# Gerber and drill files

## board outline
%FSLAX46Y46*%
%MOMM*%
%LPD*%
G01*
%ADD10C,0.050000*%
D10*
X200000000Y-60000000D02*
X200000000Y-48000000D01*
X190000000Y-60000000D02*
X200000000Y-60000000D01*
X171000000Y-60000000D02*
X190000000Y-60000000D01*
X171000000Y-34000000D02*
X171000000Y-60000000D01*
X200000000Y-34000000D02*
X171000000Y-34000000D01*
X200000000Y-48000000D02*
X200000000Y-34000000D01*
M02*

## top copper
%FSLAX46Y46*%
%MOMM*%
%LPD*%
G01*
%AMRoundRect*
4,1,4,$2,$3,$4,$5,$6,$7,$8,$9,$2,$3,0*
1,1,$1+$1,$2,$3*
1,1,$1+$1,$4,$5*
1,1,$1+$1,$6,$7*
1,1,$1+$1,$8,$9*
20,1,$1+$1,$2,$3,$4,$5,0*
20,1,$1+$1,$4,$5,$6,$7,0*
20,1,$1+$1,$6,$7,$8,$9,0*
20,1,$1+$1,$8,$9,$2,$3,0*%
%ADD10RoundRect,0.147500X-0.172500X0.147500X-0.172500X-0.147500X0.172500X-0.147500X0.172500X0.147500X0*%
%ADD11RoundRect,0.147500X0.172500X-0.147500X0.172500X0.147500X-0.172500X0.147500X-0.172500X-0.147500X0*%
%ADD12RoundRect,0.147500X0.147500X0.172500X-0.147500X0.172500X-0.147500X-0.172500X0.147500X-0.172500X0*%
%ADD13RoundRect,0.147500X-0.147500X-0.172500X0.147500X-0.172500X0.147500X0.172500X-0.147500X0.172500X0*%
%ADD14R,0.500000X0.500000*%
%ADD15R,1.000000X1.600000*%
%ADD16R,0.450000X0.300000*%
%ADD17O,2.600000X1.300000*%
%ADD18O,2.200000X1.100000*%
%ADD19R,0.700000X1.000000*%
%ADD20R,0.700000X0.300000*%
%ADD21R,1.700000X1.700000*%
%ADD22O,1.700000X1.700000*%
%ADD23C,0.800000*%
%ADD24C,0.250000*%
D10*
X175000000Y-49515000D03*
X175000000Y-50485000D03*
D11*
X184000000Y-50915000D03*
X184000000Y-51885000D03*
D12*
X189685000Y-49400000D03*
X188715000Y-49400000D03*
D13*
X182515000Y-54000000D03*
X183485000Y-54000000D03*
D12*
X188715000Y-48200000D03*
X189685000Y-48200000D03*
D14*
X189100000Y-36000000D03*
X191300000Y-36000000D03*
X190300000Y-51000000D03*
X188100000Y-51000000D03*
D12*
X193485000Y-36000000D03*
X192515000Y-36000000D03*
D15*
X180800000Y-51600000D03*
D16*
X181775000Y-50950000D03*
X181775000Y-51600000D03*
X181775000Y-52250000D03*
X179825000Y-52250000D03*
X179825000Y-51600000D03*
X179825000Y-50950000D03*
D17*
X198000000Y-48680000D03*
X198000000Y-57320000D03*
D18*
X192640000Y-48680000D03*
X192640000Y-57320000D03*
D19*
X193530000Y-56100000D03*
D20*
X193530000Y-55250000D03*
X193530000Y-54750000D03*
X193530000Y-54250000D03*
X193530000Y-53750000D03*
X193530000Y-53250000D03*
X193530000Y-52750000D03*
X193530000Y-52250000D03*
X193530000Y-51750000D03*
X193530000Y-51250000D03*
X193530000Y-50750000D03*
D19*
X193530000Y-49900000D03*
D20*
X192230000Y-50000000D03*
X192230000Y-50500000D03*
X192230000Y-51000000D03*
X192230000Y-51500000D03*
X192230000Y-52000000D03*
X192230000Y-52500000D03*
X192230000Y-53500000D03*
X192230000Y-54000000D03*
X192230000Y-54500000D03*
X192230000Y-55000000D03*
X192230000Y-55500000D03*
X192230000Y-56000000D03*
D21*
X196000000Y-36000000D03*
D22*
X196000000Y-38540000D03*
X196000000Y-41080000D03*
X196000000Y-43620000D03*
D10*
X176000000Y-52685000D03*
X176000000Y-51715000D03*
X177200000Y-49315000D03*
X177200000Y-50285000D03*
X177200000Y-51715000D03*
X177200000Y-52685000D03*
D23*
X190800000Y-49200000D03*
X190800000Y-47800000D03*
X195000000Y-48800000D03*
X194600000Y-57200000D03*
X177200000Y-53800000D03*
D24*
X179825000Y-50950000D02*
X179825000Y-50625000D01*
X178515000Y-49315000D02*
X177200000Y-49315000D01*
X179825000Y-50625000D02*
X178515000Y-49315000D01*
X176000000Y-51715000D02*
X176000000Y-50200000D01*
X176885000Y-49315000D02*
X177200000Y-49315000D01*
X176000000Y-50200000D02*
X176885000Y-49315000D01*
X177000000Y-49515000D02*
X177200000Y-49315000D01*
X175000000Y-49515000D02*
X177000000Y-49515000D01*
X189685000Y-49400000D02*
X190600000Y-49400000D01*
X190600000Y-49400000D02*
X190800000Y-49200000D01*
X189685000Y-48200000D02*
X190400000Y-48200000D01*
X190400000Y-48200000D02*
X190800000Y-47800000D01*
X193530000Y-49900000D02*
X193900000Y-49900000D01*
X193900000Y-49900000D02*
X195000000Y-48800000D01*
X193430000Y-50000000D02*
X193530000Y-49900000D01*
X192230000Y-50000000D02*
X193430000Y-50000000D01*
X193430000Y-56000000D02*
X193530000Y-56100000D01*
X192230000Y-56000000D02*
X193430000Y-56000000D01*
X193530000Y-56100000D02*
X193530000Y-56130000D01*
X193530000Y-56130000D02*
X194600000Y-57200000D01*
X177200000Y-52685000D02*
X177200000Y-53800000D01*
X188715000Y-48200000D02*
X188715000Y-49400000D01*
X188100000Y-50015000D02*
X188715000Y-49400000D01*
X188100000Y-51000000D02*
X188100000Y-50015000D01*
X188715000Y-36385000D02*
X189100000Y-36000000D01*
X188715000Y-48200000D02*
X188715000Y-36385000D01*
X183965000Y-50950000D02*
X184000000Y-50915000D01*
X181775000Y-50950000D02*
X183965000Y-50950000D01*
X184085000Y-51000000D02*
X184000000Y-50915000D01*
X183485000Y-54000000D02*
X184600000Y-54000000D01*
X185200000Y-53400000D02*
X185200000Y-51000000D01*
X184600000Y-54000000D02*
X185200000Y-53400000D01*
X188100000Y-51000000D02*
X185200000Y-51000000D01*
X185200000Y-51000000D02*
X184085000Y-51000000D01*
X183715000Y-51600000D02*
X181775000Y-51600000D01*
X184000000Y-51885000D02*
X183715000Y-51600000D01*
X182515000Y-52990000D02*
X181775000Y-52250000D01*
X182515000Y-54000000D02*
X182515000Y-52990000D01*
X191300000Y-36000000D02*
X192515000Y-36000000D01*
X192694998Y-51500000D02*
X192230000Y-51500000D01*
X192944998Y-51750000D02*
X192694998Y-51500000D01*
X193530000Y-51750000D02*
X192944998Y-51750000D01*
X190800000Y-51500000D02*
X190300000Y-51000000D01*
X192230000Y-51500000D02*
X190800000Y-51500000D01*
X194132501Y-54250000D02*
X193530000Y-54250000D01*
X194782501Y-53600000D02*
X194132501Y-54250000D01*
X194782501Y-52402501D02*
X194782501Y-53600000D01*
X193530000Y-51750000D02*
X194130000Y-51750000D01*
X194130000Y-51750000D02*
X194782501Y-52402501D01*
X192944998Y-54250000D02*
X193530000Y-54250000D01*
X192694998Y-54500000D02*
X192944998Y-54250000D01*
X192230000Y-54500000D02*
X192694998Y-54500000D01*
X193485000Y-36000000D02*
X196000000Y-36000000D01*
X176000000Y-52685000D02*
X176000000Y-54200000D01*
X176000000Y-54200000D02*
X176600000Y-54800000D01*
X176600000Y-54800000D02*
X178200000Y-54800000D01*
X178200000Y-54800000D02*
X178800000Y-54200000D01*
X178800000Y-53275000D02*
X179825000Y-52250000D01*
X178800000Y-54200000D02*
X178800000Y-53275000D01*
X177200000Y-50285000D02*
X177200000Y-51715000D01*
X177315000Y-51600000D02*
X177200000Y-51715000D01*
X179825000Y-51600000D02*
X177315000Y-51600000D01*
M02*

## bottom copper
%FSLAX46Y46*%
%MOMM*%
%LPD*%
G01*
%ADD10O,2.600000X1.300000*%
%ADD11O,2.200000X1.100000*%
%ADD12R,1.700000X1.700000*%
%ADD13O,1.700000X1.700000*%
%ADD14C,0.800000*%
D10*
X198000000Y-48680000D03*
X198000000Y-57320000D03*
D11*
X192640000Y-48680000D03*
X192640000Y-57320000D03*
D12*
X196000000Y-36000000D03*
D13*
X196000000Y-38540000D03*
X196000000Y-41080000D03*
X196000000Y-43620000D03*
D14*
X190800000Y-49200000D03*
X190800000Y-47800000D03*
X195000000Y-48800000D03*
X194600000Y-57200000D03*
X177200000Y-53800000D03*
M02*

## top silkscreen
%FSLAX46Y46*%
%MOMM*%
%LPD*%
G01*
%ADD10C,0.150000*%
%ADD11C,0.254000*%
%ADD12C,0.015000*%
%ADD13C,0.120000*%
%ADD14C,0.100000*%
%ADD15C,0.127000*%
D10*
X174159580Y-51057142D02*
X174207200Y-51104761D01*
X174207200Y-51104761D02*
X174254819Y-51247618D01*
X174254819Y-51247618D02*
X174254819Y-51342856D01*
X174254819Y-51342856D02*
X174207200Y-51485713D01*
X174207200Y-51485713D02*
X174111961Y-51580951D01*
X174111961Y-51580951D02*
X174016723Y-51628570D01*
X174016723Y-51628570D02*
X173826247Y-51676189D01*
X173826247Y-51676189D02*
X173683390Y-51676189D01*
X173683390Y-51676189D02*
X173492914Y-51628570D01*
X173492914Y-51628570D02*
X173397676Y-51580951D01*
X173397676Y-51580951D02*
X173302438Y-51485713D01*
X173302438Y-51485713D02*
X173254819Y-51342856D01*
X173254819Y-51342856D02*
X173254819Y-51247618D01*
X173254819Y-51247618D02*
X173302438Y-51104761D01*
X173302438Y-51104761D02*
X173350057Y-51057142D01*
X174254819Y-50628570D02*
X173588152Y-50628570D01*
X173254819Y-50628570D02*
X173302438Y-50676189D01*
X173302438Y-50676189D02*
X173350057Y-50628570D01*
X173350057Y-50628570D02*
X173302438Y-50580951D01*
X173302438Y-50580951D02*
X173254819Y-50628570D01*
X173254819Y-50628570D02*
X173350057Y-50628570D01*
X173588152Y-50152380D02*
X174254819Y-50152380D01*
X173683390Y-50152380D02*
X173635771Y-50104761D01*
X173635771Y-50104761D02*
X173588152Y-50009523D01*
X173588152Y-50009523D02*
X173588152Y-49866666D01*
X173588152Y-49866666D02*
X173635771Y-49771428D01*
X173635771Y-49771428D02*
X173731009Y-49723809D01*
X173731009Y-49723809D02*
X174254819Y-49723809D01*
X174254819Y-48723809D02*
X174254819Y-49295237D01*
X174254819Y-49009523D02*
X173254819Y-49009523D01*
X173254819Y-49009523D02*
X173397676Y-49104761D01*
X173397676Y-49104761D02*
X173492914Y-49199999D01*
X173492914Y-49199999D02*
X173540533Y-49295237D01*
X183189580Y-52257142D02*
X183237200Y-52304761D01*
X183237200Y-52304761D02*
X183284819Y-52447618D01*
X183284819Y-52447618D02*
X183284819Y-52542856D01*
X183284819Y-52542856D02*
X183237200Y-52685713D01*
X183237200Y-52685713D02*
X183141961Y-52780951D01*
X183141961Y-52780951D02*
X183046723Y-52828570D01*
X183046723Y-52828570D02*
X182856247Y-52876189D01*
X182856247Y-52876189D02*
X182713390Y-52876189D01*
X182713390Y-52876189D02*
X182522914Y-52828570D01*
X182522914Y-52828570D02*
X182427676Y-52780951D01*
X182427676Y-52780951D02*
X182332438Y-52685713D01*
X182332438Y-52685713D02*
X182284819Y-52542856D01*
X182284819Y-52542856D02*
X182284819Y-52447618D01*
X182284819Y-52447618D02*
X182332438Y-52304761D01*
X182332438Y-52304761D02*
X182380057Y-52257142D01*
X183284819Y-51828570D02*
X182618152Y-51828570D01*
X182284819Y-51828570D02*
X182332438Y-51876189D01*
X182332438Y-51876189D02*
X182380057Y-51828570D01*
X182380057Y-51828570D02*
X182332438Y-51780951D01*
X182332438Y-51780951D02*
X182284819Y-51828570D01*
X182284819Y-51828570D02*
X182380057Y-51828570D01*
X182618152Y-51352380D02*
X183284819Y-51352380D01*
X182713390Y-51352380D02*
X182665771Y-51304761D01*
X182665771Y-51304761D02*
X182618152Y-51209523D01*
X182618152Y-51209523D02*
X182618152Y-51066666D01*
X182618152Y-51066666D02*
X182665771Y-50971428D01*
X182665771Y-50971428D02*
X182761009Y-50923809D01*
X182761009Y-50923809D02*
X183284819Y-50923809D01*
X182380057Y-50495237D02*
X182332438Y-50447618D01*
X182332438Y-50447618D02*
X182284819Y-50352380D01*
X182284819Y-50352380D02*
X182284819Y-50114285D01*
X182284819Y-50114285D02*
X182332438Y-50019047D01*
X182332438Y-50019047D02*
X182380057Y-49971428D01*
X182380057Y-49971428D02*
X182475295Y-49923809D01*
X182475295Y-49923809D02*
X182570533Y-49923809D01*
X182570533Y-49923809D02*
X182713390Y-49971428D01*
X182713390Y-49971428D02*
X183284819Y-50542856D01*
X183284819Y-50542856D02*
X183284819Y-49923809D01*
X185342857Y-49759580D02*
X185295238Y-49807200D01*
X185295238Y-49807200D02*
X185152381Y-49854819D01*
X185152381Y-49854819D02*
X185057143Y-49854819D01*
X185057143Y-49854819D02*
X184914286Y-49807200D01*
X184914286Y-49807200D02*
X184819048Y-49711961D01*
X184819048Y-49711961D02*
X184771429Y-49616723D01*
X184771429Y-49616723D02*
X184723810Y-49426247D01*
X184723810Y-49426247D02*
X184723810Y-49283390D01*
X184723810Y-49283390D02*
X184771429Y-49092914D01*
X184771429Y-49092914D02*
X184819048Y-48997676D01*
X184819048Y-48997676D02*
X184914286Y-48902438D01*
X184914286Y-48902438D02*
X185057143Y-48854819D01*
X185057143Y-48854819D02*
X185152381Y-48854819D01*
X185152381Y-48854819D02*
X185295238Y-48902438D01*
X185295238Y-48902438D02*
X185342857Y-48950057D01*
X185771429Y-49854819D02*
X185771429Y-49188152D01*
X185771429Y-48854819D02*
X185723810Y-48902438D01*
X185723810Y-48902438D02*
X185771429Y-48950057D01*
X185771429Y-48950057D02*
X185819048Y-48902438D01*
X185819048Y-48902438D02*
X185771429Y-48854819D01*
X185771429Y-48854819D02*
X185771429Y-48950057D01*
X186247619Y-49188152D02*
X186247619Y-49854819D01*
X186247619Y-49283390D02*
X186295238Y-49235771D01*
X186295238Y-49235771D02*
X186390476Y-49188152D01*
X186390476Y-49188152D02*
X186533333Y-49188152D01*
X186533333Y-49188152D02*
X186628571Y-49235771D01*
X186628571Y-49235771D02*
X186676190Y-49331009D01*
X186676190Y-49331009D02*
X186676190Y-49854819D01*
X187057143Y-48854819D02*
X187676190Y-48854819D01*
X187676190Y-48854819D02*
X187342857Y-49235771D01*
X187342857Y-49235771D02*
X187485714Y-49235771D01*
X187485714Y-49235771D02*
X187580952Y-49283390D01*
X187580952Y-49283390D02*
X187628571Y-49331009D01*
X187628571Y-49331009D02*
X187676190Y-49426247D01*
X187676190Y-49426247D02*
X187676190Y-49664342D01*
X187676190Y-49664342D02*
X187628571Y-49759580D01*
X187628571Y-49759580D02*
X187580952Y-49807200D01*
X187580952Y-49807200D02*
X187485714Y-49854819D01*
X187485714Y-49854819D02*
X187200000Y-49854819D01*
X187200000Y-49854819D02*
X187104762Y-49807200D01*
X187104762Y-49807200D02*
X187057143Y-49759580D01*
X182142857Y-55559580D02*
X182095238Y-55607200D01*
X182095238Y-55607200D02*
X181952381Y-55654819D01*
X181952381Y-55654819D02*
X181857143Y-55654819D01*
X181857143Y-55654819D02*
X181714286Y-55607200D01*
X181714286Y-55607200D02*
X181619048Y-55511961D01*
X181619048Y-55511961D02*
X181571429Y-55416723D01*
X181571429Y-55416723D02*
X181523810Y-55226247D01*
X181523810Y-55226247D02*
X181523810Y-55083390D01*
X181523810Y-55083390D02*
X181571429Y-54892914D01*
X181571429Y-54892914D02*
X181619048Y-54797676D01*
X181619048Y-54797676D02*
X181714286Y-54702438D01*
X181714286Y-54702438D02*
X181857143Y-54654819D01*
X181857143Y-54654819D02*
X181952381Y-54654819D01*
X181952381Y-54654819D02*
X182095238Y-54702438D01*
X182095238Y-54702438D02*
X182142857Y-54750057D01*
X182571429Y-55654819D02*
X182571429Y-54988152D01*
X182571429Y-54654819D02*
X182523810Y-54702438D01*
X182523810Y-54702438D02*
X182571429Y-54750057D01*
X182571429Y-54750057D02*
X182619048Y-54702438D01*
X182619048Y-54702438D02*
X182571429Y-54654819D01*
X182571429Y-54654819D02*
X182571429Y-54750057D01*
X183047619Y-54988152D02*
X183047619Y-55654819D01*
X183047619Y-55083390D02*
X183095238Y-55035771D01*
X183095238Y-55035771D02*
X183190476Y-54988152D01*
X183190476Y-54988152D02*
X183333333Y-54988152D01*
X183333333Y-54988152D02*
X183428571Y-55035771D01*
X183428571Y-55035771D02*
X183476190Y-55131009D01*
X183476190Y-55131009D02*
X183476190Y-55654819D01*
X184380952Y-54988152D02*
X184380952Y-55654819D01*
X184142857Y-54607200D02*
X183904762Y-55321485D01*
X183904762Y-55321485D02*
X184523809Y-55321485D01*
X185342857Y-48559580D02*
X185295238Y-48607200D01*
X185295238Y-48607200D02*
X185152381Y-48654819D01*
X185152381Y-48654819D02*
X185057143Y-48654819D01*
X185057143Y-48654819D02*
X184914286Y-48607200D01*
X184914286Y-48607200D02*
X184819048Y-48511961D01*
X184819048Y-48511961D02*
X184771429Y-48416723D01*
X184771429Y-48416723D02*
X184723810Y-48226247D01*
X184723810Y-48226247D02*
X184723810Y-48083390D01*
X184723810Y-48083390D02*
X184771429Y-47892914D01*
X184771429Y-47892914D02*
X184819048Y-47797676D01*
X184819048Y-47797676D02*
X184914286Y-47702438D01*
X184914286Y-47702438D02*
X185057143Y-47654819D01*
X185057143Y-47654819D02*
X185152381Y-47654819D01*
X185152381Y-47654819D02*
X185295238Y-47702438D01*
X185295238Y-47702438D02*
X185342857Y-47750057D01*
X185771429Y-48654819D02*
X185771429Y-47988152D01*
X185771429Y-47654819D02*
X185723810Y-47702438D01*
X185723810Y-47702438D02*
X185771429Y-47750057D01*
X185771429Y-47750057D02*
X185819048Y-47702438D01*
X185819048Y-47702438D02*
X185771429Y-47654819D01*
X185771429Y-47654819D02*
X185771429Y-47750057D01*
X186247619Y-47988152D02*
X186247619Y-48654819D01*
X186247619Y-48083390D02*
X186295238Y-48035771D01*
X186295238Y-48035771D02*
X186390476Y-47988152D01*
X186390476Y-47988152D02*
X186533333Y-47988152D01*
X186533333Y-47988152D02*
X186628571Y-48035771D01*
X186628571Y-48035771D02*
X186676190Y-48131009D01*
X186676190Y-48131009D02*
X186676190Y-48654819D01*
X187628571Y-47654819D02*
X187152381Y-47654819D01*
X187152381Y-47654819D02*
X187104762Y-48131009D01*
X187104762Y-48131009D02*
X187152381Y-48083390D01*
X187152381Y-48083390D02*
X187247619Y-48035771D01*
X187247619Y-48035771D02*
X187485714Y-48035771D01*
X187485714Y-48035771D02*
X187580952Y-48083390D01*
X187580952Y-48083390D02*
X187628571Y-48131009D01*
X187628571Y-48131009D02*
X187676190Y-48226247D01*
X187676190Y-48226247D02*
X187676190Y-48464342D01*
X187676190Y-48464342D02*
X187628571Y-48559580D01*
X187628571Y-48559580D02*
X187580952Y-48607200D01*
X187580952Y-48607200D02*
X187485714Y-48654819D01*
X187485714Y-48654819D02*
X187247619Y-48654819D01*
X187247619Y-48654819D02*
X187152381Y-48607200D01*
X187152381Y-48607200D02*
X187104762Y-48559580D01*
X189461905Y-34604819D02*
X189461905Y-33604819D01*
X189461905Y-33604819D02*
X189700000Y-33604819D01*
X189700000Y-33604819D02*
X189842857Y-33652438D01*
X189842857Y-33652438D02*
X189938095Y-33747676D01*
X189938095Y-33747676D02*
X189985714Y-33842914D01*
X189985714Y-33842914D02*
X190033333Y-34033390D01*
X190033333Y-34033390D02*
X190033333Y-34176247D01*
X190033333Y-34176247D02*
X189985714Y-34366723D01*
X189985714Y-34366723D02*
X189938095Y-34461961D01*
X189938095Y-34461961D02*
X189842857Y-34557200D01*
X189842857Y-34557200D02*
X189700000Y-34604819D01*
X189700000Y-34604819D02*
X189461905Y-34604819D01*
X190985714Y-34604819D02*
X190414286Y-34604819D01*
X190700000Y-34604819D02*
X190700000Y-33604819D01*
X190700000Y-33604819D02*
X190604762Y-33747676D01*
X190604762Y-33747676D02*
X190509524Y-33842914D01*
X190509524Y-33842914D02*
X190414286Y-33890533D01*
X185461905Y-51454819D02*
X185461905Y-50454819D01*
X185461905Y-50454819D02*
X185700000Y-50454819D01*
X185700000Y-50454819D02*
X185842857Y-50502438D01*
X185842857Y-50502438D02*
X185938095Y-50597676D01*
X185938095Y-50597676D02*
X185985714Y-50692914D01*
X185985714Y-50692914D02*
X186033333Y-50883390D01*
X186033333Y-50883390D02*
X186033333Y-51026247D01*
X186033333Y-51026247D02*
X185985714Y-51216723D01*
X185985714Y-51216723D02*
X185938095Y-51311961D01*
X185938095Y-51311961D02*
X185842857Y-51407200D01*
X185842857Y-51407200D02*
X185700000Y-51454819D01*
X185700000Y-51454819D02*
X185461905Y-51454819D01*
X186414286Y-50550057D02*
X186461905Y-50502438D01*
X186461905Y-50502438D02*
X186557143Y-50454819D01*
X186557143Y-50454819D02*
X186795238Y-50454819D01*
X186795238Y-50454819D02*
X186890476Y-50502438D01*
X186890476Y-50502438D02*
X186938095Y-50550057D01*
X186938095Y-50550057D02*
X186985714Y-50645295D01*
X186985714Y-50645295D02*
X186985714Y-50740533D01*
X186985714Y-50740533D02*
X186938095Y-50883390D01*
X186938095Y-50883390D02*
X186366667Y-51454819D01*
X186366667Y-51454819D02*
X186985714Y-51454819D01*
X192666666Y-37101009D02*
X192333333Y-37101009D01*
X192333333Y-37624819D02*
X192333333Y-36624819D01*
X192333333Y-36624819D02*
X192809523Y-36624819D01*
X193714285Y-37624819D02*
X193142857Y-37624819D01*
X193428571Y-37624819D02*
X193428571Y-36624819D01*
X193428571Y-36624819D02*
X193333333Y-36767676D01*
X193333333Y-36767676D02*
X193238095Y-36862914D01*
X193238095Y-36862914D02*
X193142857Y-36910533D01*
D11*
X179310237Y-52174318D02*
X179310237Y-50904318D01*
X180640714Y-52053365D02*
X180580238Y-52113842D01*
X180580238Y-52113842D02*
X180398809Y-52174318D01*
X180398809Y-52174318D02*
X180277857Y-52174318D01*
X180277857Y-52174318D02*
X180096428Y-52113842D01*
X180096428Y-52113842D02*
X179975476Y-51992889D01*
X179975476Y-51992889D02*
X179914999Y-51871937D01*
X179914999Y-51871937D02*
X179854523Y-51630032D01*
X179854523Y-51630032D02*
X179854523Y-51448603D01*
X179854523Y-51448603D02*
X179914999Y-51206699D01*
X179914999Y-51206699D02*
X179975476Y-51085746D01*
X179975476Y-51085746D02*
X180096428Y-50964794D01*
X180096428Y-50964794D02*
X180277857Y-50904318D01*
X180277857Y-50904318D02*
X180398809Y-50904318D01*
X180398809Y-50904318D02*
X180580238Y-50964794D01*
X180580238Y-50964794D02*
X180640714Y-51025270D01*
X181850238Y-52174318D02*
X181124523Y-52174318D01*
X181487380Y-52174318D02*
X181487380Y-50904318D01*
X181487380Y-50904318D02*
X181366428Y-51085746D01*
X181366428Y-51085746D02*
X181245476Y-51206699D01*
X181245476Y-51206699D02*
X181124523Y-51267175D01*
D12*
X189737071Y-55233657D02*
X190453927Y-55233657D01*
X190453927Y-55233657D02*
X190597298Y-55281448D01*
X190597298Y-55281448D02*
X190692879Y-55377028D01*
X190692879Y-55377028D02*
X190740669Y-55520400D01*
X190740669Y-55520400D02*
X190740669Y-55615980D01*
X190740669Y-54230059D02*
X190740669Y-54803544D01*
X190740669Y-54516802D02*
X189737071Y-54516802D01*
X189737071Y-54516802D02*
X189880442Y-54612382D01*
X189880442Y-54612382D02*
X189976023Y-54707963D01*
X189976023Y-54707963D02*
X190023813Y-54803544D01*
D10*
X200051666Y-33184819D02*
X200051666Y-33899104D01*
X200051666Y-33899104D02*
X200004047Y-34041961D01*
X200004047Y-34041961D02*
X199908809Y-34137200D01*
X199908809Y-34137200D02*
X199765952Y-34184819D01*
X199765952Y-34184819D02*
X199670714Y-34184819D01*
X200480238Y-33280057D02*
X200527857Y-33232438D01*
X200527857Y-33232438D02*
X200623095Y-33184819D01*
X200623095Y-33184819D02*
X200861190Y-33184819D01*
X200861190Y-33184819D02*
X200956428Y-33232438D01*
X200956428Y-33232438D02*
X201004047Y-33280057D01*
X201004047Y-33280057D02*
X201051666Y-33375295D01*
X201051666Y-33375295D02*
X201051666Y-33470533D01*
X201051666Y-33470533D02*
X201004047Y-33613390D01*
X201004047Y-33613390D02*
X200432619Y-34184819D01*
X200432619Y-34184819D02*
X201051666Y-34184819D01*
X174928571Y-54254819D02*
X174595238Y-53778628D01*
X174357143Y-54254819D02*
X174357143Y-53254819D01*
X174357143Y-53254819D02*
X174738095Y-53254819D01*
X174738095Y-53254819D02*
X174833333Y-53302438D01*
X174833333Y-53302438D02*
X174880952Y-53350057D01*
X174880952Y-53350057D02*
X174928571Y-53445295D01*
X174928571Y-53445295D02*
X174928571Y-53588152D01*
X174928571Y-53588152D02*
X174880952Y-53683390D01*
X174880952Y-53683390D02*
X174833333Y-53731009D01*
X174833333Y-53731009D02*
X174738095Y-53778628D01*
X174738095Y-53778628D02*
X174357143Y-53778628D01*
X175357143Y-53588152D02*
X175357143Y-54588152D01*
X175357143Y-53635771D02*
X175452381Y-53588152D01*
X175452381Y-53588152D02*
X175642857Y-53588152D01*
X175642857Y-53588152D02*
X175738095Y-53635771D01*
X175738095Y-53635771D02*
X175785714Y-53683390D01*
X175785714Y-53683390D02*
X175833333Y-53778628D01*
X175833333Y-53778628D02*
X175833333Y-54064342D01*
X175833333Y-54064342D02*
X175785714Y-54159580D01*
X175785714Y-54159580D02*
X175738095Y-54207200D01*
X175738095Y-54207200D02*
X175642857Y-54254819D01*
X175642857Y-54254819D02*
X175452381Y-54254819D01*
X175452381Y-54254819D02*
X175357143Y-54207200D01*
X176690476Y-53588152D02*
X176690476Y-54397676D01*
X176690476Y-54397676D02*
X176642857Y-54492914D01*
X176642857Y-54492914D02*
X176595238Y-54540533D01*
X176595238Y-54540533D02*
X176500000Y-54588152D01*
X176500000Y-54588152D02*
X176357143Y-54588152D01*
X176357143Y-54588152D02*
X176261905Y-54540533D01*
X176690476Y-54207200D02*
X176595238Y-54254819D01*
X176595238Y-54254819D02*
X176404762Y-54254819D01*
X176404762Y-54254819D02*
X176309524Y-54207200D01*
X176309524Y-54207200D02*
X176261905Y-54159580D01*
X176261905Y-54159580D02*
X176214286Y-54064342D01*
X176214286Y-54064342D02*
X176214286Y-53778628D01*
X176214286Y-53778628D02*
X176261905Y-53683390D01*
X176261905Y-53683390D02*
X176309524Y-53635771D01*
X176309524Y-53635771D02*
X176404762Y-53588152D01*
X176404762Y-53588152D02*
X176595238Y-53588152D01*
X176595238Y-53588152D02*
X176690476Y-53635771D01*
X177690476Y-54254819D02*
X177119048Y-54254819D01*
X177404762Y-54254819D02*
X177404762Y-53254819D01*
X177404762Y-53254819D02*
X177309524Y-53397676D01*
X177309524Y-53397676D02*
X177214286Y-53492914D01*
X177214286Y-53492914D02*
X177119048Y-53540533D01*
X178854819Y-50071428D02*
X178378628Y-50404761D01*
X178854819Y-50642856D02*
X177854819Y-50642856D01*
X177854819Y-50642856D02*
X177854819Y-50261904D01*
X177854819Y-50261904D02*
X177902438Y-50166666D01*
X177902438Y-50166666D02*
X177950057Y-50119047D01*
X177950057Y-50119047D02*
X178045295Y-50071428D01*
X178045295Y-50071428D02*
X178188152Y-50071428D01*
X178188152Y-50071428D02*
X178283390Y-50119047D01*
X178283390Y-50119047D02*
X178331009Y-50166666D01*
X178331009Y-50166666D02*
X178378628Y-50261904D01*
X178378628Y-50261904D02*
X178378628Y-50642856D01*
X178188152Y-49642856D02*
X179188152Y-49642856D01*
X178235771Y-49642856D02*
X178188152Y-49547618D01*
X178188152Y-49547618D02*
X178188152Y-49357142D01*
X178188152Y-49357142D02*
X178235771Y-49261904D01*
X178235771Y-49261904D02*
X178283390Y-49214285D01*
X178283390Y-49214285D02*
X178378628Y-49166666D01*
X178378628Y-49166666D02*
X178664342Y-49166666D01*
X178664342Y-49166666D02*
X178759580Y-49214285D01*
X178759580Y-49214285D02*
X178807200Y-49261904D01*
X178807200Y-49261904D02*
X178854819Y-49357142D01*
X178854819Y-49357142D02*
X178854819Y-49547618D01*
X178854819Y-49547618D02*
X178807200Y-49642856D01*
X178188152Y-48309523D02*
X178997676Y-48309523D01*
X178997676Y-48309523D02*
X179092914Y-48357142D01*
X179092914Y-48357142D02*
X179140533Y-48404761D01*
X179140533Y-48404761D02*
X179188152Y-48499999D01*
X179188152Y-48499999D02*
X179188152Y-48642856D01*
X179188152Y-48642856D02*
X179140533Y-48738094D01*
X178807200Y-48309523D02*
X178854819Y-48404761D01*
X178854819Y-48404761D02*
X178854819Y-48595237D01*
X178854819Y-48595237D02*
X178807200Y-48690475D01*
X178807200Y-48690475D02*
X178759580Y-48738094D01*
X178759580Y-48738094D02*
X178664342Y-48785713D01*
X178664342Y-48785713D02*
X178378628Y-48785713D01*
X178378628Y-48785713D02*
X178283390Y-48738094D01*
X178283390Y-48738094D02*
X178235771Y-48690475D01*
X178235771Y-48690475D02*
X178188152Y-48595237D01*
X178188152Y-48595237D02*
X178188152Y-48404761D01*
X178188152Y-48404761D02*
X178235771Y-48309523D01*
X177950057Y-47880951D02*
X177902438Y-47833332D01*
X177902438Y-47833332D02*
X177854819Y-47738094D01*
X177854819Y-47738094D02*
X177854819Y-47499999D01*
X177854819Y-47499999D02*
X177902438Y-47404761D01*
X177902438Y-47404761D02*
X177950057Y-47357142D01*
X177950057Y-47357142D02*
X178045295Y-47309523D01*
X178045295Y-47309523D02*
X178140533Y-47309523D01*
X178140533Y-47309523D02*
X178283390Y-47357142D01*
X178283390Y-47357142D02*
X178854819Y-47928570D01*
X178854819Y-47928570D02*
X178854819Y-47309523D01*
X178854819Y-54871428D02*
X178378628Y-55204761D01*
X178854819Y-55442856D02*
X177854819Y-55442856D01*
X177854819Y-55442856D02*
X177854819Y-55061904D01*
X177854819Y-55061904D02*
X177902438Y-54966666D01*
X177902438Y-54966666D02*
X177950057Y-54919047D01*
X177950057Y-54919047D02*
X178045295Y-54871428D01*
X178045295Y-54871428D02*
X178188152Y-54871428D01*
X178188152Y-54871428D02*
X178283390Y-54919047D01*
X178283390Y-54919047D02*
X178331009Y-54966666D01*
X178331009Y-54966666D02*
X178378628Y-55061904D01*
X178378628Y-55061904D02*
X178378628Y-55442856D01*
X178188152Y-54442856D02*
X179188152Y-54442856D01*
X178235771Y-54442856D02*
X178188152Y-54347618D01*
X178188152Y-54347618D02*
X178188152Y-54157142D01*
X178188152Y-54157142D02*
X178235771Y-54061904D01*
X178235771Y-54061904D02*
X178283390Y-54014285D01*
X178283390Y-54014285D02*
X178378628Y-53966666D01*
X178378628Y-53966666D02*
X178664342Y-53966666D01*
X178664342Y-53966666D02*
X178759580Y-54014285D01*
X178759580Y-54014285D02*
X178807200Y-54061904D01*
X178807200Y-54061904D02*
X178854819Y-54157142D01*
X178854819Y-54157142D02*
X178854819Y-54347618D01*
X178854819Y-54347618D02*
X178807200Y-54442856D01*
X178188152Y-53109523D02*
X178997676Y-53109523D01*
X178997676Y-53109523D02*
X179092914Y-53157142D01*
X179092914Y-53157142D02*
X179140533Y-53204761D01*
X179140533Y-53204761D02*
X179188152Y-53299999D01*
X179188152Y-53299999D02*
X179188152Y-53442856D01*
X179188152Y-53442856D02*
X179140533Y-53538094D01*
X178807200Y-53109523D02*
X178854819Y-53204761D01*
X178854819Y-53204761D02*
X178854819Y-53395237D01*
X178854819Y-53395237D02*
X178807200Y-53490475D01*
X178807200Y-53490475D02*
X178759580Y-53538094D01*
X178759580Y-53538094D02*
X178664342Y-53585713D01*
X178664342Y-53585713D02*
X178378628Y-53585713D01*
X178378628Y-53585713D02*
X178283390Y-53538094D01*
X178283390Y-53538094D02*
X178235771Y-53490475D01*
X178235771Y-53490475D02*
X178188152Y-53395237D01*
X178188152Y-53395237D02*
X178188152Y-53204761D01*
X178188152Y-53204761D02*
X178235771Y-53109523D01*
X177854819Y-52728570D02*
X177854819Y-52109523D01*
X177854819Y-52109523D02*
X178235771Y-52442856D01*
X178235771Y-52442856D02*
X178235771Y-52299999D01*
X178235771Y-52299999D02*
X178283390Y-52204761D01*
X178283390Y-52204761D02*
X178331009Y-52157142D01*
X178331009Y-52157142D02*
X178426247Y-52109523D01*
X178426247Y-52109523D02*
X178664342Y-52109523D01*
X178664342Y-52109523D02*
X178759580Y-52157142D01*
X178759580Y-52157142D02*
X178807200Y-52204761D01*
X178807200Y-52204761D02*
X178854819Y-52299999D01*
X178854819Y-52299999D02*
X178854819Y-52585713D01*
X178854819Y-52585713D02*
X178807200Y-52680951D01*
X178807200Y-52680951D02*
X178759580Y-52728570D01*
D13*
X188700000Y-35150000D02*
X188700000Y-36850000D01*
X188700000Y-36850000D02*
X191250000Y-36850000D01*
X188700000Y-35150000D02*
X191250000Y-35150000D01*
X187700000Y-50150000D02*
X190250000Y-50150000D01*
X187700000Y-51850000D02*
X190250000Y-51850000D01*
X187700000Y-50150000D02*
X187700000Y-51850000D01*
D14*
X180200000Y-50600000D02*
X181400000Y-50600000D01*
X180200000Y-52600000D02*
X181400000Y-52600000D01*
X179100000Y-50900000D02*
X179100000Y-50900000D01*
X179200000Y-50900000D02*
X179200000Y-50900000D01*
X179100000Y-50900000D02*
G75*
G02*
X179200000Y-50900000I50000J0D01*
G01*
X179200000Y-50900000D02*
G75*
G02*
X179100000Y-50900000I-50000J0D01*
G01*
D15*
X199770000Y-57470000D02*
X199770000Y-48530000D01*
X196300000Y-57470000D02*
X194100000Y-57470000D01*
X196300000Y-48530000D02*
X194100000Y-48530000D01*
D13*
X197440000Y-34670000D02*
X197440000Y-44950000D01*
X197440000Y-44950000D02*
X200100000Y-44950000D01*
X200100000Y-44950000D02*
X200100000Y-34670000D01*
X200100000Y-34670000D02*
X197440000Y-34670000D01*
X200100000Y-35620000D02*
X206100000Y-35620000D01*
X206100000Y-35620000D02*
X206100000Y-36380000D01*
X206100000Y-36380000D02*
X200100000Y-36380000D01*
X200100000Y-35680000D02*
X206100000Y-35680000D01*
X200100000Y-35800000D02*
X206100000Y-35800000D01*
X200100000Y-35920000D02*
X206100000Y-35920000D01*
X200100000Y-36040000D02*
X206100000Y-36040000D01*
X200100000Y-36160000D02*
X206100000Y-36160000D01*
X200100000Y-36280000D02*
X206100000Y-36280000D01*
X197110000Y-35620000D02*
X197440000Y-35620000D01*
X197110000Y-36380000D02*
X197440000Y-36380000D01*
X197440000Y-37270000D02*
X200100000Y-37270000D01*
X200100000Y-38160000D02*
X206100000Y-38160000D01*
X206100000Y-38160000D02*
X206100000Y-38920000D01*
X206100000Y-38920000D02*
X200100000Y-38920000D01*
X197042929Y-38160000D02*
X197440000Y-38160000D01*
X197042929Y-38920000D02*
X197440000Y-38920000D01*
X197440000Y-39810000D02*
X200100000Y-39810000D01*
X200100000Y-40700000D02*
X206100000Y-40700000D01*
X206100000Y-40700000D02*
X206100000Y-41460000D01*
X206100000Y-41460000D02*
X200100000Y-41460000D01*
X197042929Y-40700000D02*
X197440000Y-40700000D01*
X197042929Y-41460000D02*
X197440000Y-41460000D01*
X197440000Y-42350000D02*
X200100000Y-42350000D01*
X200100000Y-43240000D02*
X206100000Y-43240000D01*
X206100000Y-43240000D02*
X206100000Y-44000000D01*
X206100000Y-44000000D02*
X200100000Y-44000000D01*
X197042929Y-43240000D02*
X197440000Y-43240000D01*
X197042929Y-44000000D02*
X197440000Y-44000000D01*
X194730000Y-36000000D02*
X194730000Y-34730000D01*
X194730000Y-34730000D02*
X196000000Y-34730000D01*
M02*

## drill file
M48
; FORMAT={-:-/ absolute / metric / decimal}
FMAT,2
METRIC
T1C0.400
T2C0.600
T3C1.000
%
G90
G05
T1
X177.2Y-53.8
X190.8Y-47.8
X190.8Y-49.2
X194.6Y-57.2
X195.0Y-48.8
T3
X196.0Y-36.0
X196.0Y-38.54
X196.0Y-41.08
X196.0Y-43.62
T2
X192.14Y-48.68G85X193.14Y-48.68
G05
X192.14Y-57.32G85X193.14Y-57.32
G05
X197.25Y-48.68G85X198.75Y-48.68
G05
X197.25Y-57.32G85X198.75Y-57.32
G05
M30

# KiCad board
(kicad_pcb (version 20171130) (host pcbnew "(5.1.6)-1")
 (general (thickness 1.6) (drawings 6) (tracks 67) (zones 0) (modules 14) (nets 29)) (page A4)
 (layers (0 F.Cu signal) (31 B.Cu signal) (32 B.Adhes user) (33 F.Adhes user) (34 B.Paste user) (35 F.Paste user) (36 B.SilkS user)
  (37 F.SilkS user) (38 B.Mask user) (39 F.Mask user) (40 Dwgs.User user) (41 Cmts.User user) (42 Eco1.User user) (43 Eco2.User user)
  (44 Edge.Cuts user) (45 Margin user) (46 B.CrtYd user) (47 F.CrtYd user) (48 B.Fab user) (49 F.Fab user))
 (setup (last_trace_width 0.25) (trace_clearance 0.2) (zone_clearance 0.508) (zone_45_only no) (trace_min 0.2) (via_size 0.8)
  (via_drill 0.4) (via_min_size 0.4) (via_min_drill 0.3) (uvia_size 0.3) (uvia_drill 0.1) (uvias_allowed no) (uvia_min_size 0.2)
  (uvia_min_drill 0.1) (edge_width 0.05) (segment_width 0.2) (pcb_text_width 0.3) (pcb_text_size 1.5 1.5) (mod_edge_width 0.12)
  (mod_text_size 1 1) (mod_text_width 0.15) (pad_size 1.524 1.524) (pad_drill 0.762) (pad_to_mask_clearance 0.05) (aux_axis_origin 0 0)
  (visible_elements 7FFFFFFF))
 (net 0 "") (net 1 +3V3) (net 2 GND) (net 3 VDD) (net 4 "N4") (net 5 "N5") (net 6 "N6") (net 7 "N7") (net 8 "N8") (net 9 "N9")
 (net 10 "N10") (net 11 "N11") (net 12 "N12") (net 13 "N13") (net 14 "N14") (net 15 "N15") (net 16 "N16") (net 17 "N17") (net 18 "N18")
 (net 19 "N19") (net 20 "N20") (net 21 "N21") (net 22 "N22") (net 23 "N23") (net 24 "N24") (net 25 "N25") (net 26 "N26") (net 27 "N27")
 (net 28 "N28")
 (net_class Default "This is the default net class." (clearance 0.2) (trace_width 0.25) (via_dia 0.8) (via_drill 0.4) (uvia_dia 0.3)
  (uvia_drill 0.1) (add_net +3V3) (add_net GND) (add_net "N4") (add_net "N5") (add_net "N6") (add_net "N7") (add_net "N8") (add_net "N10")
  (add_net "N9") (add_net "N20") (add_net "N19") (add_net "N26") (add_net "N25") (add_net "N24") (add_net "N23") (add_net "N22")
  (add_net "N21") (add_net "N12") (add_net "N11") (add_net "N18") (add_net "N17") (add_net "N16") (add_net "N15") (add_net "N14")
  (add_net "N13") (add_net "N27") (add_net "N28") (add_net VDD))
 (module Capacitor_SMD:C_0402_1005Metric (layer F.Cu) (at 175 50 270)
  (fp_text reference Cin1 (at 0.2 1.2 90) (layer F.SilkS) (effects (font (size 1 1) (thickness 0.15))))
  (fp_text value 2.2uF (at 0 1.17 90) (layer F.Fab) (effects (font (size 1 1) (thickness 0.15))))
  (pad 1 smd roundrect (at -0.485 0 270) (size 0.59 0.64) (layers F.Cu F.Paste F.Mask) (roundrect_rratio 0.25) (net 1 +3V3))
  (pad 2 smd roundrect (at 0.485 0 270) (size 0.59 0.64) (layers F.Cu F.Paste F.Mask) (roundrect_rratio 0.25) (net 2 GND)))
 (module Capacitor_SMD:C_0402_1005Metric (layer F.Cu) (at 184 51.4 90)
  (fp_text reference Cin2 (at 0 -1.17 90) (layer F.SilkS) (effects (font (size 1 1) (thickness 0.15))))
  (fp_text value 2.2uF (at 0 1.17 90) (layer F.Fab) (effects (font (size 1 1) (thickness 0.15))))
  (pad 2 smd roundrect (at 0.485 0 90) (size 0.59 0.64) (layers F.Cu F.Paste F.Mask) (roundrect_rratio 0.25) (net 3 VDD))
  (pad 1 smd roundrect (at -0.485 0 90) (size 0.59 0.64) (layers F.Cu F.Paste F.Mask) (roundrect_rratio 0.25) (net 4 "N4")))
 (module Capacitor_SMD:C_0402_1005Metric (layer F.Cu) (at 189.2 49.4 180)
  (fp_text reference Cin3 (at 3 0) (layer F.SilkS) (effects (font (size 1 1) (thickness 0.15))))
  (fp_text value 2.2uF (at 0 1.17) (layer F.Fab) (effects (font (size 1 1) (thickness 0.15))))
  (pad 1 smd roundrect (at -0.485 0 180) (size 0.59 0.64) (layers F.Cu F.Paste F.Mask) (roundrect_rratio 0.25) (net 2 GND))
  (pad 2 smd roundrect (at 0.485 0 180) (size 0.59 0.64) (layers F.Cu F.Paste F.Mask) (roundrect_rratio 0.25) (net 3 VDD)))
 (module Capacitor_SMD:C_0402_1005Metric (layer F.Cu) (at 183 54)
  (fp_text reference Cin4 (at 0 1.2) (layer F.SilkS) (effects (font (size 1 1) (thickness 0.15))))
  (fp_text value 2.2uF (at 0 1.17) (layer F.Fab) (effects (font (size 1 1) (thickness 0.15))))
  (pad 1 smd roundrect (at -0.485 0) (size 0.59 0.64) (layers F.Cu F.Paste F.Mask) (roundrect_rratio 0.25) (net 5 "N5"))
  (pad 2 smd roundrect (at 0.485 0) (size 0.59 0.64) (layers F.Cu F.Paste F.Mask) (roundrect_rratio 0.25) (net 3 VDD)))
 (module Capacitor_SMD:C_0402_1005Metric (layer F.Cu) (at 189.2 48.2 180)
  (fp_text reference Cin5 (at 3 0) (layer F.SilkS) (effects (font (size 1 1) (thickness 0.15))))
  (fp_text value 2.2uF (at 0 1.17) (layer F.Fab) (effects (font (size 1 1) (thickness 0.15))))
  (pad 2 smd roundrect (at 0.485 0 180) (size 0.59 0.64) (layers F.Cu F.Paste F.Mask) (roundrect_rratio 0.25) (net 3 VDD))
  (pad 1 smd roundrect (at -0.485 0 180) (size 0.59 0.64) (layers F.Cu F.Paste F.Mask) (roundrect_rratio 0.25) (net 2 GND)))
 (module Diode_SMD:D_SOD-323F (layer F.Cu) (at 190.2 36)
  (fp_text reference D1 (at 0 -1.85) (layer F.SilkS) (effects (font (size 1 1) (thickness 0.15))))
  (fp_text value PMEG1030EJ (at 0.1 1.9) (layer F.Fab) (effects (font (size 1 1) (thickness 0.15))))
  (fp_line (start -1.5 -0.85) (end -1.5 0.85) (layer F.SilkS) (width 0.12))
  (fp_line (start -1.5 0.85) (end 1.05 0.85) (layer F.SilkS) (width 0.12))
  (fp_line (start -1.5 -0.85) (end 1.05 -0.85) (layer F.SilkS) (width 0.12))
  (pad 1 smd rect (at -1.1 0) (size 0.5 0.5) (layers F.Cu F.Paste F.Mask) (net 3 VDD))
  (pad 2 smd rect (at 1.1 0) (size 0.5 0.5) (layers F.Cu F.Paste F.Mask) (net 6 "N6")))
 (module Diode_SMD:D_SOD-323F (layer F.Cu) (at 189.2 51)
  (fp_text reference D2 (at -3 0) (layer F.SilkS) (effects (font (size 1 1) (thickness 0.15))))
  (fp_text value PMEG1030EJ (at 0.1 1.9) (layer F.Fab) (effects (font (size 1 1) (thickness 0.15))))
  (fp_line (start -1.5 -0.85) (end 1.05 -0.85) (layer F.SilkS) (width 0.12))
  (fp_line (start -1.5 0.85) (end 1.05 0.85) (layer F.SilkS) (width 0.12))
  (fp_line (start -1.5 -0.85) (end -1.5 0.85) (layer F.SilkS) (width 0.12))
  (pad 2 smd rect (at 1.1 0) (size 0.5 0.5) (layers F.Cu F.Paste F.Mask) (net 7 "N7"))
  (pad 1 smd rect (at -1.1 0) (size 0.5 0.5) (layers F.Cu F.Paste F.Mask) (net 3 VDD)))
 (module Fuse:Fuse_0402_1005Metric (layer F.Cu) (at 193 36 180)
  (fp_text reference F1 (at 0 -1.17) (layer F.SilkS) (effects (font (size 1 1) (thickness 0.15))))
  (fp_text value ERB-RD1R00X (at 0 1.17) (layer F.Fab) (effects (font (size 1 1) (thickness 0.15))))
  (pad 1 smd roundrect (at -0.485 0 180) (size 0.59 0.64) (layers F.Cu F.Paste F.Mask) (roundrect_rratio 0.25) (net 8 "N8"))
  (pad 2 smd roundrect (at 0.485 0 180) (size 0.59 0.64) (layers F.Cu F.Paste F.Mask) (roundrect_rratio 0.25) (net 6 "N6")))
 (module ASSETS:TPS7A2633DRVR (layer F.Cu) (at 180.8 51.6)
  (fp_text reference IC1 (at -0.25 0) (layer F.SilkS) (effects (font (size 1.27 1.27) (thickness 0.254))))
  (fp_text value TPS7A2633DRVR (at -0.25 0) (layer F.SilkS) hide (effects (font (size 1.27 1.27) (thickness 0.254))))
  (fp_line (start -0.6 -1) (end 0.6 -1) (layer F.SilkS) (width 0.1))
  (fp_line (start -0.6 1) (end 0.6 1) (layer F.SilkS) (width 0.1))
  (fp_line (start -1.7 -0.7) (end -1.7 -0.7) (layer F.SilkS) (width 0.1))
  (fp_line (start -1.6 -0.7) (end -1.6 -0.7) (layer F.SilkS) (width 0.1))
  (fp_arc (start -1.65 -0.7) (end -1.6 -0.7) (angle -180) (layer F.SilkS) (width 0.1))
  (fp_arc (start -1.65 -0.7) (end -1.7 -0.7) (angle -180) (layer F.SilkS) (width 0.1))
  (pad 7 smd rect (at 0 0) (size 1 1.6) (layers F.Cu F.Paste F.Mask) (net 2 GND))
  (pad 6 smd rect (at 0.975 -0.65 90) (size 0.3 0.45) (layers F.Cu F.Paste F.Mask) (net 3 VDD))
  (pad 5 smd rect (at 0.975 0 90) (size 0.3 0.45) (layers F.Cu F.Paste F.Mask) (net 4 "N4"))
  (pad 4 smd rect (at 0.975 0.65 90) (size 0.3 0.45) (layers F.Cu F.Paste F.Mask) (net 5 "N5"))
  (pad 3 smd rect (at -0.975 0.65 90) (size 0.3 0.45) (layers F.Cu F.Paste F.Mask) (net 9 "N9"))
  (pad 2 smd rect (at -0.975 0 90) (size 0.3 0.45) (layers F.Cu F.Paste F.Mask) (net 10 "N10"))
  (pad 1 smd rect (at -0.975 -0.65 90) (size 0.3 0.45) (layers F.Cu F.Paste F.Mask) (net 1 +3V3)))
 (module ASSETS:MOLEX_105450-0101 (layer F.Cu) (at 196 53 90)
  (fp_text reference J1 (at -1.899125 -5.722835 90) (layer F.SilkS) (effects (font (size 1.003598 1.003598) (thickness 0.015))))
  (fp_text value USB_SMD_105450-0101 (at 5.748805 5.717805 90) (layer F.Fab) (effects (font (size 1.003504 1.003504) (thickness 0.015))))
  (fp_line (start -4.47 3.77) (end 4.47 3.77) (layer F.SilkS) (width 0.127))
  (fp_line (start -4.47 0.3) (end -4.47 -1.9) (layer F.SilkS) (width 0.127))
  (fp_line (start 4.47 0.3) (end 4.47 -1.9) (layer F.SilkS) (width 0.127))
  (pad S4 thru_hole oval (at 4.32 2 90) (size 1.3 2.6) (drill oval 0.6 2.1) (layers *.Cu *.Mask) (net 2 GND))
  (pad S3 thru_hole oval (at -4.32 2 90) (size 1.3 2.6) (drill oval 0.6 2.1) (layers *.Cu *.Mask) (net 2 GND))
  (pad S2 thru_hole oval (at 4.32 -3.36 90) (size 1.1 2.2) (drill oval 0.6 1.6) (layers *.Cu *.Mask) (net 2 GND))
  (pad S1 thru_hole oval (at -4.32 -3.36 90) (size 1.1 2.2) (drill oval 0.6 1.6) (layers *.Cu *.Mask) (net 2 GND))
  (pad B12 smd rect (at -3.1 -2.47 90) (size 1 0.7) (layers F.Cu F.Paste F.Mask) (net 2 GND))
  (pad B11 smd rect (at -2.25 -2.47 90) (size 0.3 0.7) (layers F.Cu F.Paste F.Mask) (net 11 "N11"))
  (pad B10 smd rect (at -1.75 -2.47 90) (size 0.3 0.7) (layers F.Cu F.Paste F.Mask) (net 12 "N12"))
  (pad B9 smd rect (at -1.25 -2.47 90) (size 0.3 0.7) (layers F.Cu F.Paste F.Mask) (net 7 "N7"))
  (pad B8 smd rect (at -0.75 -2.47 90) (size 0.3 0.7) (layers F.Cu F.Paste F.Mask) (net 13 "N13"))
  (pad B7 smd rect (at -0.25 -2.47 90) (size 0.3 0.7) (layers F.Cu F.Paste F.Mask) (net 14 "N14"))
  (pad B6 smd rect (at 0.25 -2.47 90) (size 0.3 0.7) (layers F.Cu F.Paste F.Mask) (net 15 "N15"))
  (pad B5 smd rect (at 0.75 -2.47 90) (size 0.3 0.7) (layers F.Cu F.Paste F.Mask) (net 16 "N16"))
  (pad B4 smd rect (at 1.25 -2.47 90) (size 0.3 0.7) (layers F.Cu F.Paste F.Mask) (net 7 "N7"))
  (pad B3 smd rect (at 1.75 -2.47 90) (size 0.3 0.7) (layers F.Cu F.Paste F.Mask) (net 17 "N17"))
  (pad B2 smd rect (at 2.25 -2.47 90) (size 0.3 0.7) (layers F.Cu F.Paste F.Mask) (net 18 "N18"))
  (pad B1 smd rect (at 3.1 -2.47 90) (size 1 0.7) (layers F.Cu F.Paste F.Mask) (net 2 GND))
  (pad A12 smd rect (at 3 -3.77 90) (size 0.3 0.7) (layers F.Cu F.Paste F.Mask) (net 2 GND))
  (pad A11 smd rect (at 2.5 -3.77 90) (size 0.3 0.7) (layers F.Cu F.Paste F.Mask) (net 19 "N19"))
  (pad A10 smd rect (at 2 -3.77 90) (size 0.3 0.7) (layers F.Cu F.Paste F.Mask) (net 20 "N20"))
  (pad A9 smd rect (at 1.5 -3.77 90) (size 0.3 0.7) (layers F.Cu F.Paste F.Mask) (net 7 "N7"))
  (pad A8 smd rect (at 1 -3.77 90) (size 0.3 0.7) (layers F.Cu F.Paste F.Mask) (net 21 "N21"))
  (pad A7 smd rect (at 0.5 -3.77 90) (size 0.3 0.7) (layers F.Cu F.Paste F.Mask) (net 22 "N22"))
  (pad A6 smd rect (at -0.5 -3.77 90) (size 0.3 0.7) (layers F.Cu F.Paste F.Mask) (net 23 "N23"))
  (pad A5 smd rect (at -1 -3.77 90) (size 0.3 0.7) (layers F.Cu F.Paste F.Mask) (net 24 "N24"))
  (pad A4 smd rect (at -1.5 -3.77 90) (size 0.3 0.7) (layers F.Cu F.Paste F.Mask) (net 7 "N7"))
  (pad A3 smd rect (at -2 -3.77 90) (size 0.3 0.7) (layers F.Cu F.Paste F.Mask) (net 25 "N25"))
  (pad A2 smd rect (at -2.5 -3.77 90) (size 0.3 0.7) (layers F.Cu F.Paste F.Mask) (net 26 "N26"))
  (pad A1 smd rect (at -3 -3.77 90) (size 0.3 0.7) (layers F.Cu F.Paste F.Mask) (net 2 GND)))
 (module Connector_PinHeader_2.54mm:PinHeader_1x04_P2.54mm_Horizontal (layer F.Cu) (at 196 36)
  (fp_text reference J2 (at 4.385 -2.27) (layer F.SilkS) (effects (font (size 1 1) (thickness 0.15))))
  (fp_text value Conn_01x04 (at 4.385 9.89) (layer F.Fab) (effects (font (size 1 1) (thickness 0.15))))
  (fp_line (start 1.44 -1.33) (end 1.44 8.95) (layer F.SilkS) (width 0.12))
  (fp_line (start 1.44 8.95) (end 4.1 8.95) (layer F.SilkS) (width 0.12))
  (fp_line (start 4.1 8.95) (end 4.1 -1.33) (layer F.SilkS) (width 0.12))
  (fp_line (start 4.1 -1.33) (end 1.44 -1.33) (layer F.SilkS) (width 0.12))
  (fp_line (start 4.1 -0.38) (end 10.1 -0.38) (layer F.SilkS) (width 0.12))
  (fp_line (start 10.1 -0.38) (end 10.1 0.38) (layer F.SilkS) (width 0.12))
  (fp_line (start 10.1 0.38) (end 4.1 0.38) (layer F.SilkS) (width 0.12))
  (fp_line (start 4.1 -0.32) (end 10.1 -0.32) (layer F.SilkS) (width 0.12))
  (fp_line (start 4.1 -0.2) (end 10.1 -0.2) (layer F.SilkS) (width 0.12))
  (fp_line (start 4.1 -0.08) (end 10.1 -0.08) (layer F.SilkS) (width 0.12))
  (fp_line (start 4.1 0.04) (end 10.1 0.04) (layer F.SilkS) (width 0.12))
  (fp_line (start 4.1 0.16) (end 10.1 0.16) (layer F.SilkS) (width 0.12))
  (fp_line (start 4.1 0.28) (end 10.1 0.28) (layer F.SilkS) (width 0.12))
  (fp_line (start 1.11 -0.38) (end 1.44 -0.38) (layer F.SilkS) (width 0.12))
  (fp_line (start 1.11 0.38) (end 1.44 0.38) (layer F.SilkS) (width 0.12))
  (fp_line (start 1.44 1.27) (end 4.1 1.27) (layer F.SilkS) (width 0.12))
  (fp_line (start 4.1 2.16) (end 10.1 2.16) (layer F.SilkS) (width 0.12))
  (fp_line (start 10.1 2.16) (end 10.1 2.92) (layer F.SilkS) (width 0.12))
  (fp_line (start 10.1 2.92) (end 4.1 2.92) (layer F.SilkS) (width 0.12))
  (fp_line (start 1.042929 2.16) (end 1.44 2.16) (layer F.SilkS) (width 0.12))
  (fp_line (start 1.042929 2.92) (end 1.44 2.92) (layer F.SilkS) (width 0.12))
  (fp_line (start 1.44 3.81) (end 4.1 3.81) (layer F.SilkS) (width 0.12))
  (fp_line (start 4.1 4.7) (end 10.1 4.7) (layer F.SilkS) (width 0.12))
  (fp_line (start 10.1 4.7) (end 10.1 5.46) (layer F.SilkS) (width 0.12))
  (fp_line (start 10.1 5.46) (end 4.1 5.46) (layer F.SilkS) (width 0.12))
  (fp_line (start 1.042929 4.7) (end 1.44 4.7) (layer F.SilkS) (width 0.12))
  (fp_line (start 1.042929 5.46) (end 1.44 5.46) (layer F.SilkS) (width 0.12))
  (fp_line (start 1.44 6.35) (end 4.1 6.35) (layer F.SilkS) (width 0.12))
  (fp_line (start 4.1 7.24) (end 10.1 7.24) (layer F.SilkS) (width 0.12))
  (fp_line (start 10.1 7.24) (end 10.1 8) (layer F.SilkS) (width 0.12))
  (fp_line (start 10.1 8) (end 4.1 8) (layer F.SilkS) (width 0.12))
  (fp_line (start 1.042929 7.24) (end 1.44 7.24) (layer F.SilkS) (width 0.12))
  (fp_line (start 1.042929 8) (end 1.44 8) (layer F.SilkS) (width 0.12))
  (fp_line (start -1.27 0) (end -1.27 -1.27) (layer F.SilkS) (width 0.12))
  (fp_line (start -1.27 -1.27) (end 0 -1.27) (layer F.SilkS) (width 0.12))
  (pad 1 thru_hole rect (at 0 0) (size 1.7 1.7) (drill 1) (layers *.Cu *.Mask) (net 8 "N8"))
  (pad 2 thru_hole oval (at 0 2.54) (size 1.7 1.7) (drill 1) (layers *.Cu *.Mask) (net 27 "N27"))
  (pad 3 thru_hole oval (at 0 5.08) (size 1.7 1.7) (drill 1) (layers *.Cu *.Mask) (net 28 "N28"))
  (pad 4 thru_hole oval (at 0 7.62) (size 1.7 1.7) (drill 1) (layers *.Cu *.Mask) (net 2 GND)))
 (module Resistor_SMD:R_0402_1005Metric (layer F.Cu) (at 176 52.2 270)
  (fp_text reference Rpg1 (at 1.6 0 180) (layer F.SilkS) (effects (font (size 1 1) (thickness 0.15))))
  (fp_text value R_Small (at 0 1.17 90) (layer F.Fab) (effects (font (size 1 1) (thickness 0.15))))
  (pad 2 smd roundrect (at 0.485 0 270) (size 0.59 0.64) (layers F.Cu F.Paste F.Mask) (roundrect_rratio 0.25) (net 9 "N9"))
  (pad 1 smd roundrect (at -0.485 0 270) (size 0.59 0.64) (layers F.Cu F.Paste F.Mask) (roundrect_rratio 0.25) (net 1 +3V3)))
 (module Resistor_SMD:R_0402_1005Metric (layer F.Cu) (at 177.2 49.8 270)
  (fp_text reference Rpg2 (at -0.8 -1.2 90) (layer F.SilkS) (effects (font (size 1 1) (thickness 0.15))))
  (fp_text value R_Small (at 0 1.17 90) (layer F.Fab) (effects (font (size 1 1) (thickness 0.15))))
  (pad 1 smd roundrect (at -0.485 0 270) (size 0.59 0.64) (layers F.Cu F.Paste F.Mask) (roundrect_rratio 0.25) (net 1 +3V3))
  (pad 2 smd roundrect (at 0.485 0 270) (size 0.59 0.64) (layers F.Cu F.Paste F.Mask) (roundrect_rratio 0.25) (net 10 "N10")))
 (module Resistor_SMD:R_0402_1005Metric (layer F.Cu) (at 177.2 52.2 270)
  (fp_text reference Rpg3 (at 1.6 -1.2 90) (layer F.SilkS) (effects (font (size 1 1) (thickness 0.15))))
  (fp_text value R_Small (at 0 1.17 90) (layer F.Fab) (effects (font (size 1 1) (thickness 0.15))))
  (pad 1 smd roundrect (at -0.485 0 270) (size 0.59 0.64) (layers F.Cu F.Paste F.Mask) (roundrect_rratio 0.25) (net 10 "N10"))
  (pad 2 smd roundrect (at 0.485 0 270) (size 0.59 0.64) (layers F.Cu F.Paste F.Mask) (roundrect_rratio 0.25) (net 2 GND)))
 (gr_line (start 200 60) (end 200 48) (layer Edge.Cuts) (width 0.05))
 (gr_line (start 190 60) (end 200 60) (layer Edge.Cuts) (width 0.05))
 (gr_line (start 171 60) (end 190 60) (layer Edge.Cuts) (width 0.05))
 (gr_line (start 171 34) (end 171 60) (layer Edge.Cuts) (width 0.05))
 (gr_line (start 200 34) (end 171 34) (layer Edge.Cuts) (width 0.05))
 (gr_line (start 200 48) (end 200 34) (layer Edge.Cuts) (width 0.05))
 (segment (start 179.825 50.95) (end 179.825 50.625) (width 0.25) (layer F.Cu) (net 1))
 (segment (start 178.515 49.315) (end 177.2 49.315) (width 0.25) (layer F.Cu) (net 1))
 (segment (start 179.825 50.625) (end 178.515 49.315) (width 0.25) (layer F.Cu) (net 1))
 (segment (start 176 51.715) (end 176 50.2) (width 0.25) (layer F.Cu) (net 1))
 (segment (start 176.885 49.315) (end 177.2 49.315) (width 0.25) (layer F.Cu) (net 1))
 (segment (start 176 50.2) (end 176.885 49.315) (width 0.25) (layer F.Cu) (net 1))
 (segment (start 177 49.515) (end 177.2 49.315) (width 0.25) (layer F.Cu) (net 1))
 (segment (start 175 49.515) (end 177 49.515) (width 0.25) (layer F.Cu) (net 1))
 (via (at 190.8 49.2) (size 0.8) (drill 0.4) (layers F.Cu B.Cu) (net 2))
 (segment (start 189.685 49.4) (end 190.6 49.4) (width 0.25) (layer F.Cu) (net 2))
 (segment (start 190.6 49.4) (end 190.8 49.2) (width 0.25) (layer F.Cu) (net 2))
 (via (at 190.8 47.8) (size 0.8) (drill 0.4) (layers F.Cu B.Cu) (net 2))
 (segment (start 189.685 48.2) (end 190.4 48.2) (width 0.25) (layer F.Cu) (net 2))
 (segment (start 190.4 48.2) (end 190.8 47.8) (width 0.25) (layer F.Cu) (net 2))
 (segment (start 193.53 49.9) (end 193.9 49.9) (width 0.25) (layer F.Cu) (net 2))
 (via (at 195 48.8) (size 0.8) (drill 0.4) (layers F.Cu B.Cu) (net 2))
 (segment (start 193.9 49.9) (end 195 48.8) (width 0.25) (layer F.Cu) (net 2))
 (segment (start 193.43 50) (end 193.53 49.9) (width 0.25) (layer F.Cu) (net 2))
 (segment (start 192.23 50) (end 193.43 50) (width 0.25) (layer F.Cu) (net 2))
 (segment (start 193.43 56) (end 193.53 56.1) (width 0.25) (layer F.Cu) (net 2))
 (segment (start 192.23 56) (end 193.43 56) (width 0.25) (layer F.Cu) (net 2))
 (via (at 194.6 57.2) (size 0.8) (drill 0.4) (layers F.Cu B.Cu) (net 2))
 (segment (start 193.53 56.1) (end 193.53 56.13) (width 0.25) (layer F.Cu) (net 2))
 (segment (start 193.53 56.13) (end 194.6 57.2) (width 0.25) (layer F.Cu) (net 2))
 (via (at 177.2 53.8) (size 0.8) (drill 0.4) (layers F.Cu B.Cu) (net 2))
 (segment (start 177.2 52.685) (end 177.2 53.8) (width 0.25) (layer F.Cu) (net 2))
 (segment (start 188.715 48.2) (end 188.715 49.4) (width 0.25) (layer F.Cu) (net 3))
 (segment (start 188.1 50.015) (end 188.715 49.4) (width 0.25) (layer F.Cu) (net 3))
 (segment (start 188.1 51) (end 188.1 50.015) (width 0.25) (layer F.Cu) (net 3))
 (segment (start 188.715 36.385) (end 189.1 36) (width 0.25) (layer F.Cu) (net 3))
 (segment (start 188.715 48.2) (end 188.715 36.385) (width 0.25) (layer F.Cu) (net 3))
 (segment (start 183.965 50.95) (end 184 50.915) (width 0.25) (layer F.Cu) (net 3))
 (segment (start 181.775 50.95) (end 183.965 50.95) (width 0.25) (layer F.Cu) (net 3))
 (segment (start 184.085 51) (end 184 50.915) (width 0.25) (layer F.Cu) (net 3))
 (segment (start 183.485 54) (end 184.6 54) (width 0.25) (layer F.Cu) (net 3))
 (segment (start 185.2 53.4) (end 185.2 51) (width 0.25) (layer F.Cu) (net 3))
 (segment (start 184.6 54) (end 185.2 53.4) (width 0.25) (layer F.Cu) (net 3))
 (segment (start 188.1 51) (end 185.2 51) (width 0.25) (layer F.Cu) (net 3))
 (segment (start 185.2 51) (end 184.085 51) (width 0.25) (layer F.Cu) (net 3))
 (segment (start 183.715 51.6) (end 181.775 51.6) (width 0.25) (layer F.Cu) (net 4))
 (segment (start 184 51.885) (end 183.715 51.6) (width 0.25) (layer F.Cu) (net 4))
 (segment (start 182.515 52.99) (end 181.775 52.25) (width 0.25) (layer F.Cu) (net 5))
 (segment (start 182.515 54) (end 182.515 52.99) (width 0.25) (layer F.Cu) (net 5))
 (segment (start 191.3 36) (end 192.515 36) (width 0.25) (layer F.Cu) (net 6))
 (segment (start 192.694998 51.5) (end 192.23 51.5) (width 0.25) (layer F.Cu) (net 7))
 (segment (start 192.944998 51.75) (end 192.694998 51.5) (width 0.25) (layer F.Cu) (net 7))
 (segment (start 193.53 51.75) (end 192.944998 51.75) (width 0.25) (layer F.Cu) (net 7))
 (segment (start 190.8 51.5) (end 190.3 51) (width 0.25) (layer F.Cu) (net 7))
 (segment (start 192.23 51.5) (end 190.8 51.5) (width 0.25) (layer F.Cu) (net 7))
 (segment (start 194.132501 54.25) (end 193.53 54.25) (width 0.25) (layer F.Cu) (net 7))
 (segment (start 194.782501 53.6) (end 194.132501 54.25) (width 0.25) (layer F.Cu) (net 7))
 (segment (start 194.782501 52.402501) (end 194.782501 53.6) (width 0.25) (layer F.Cu) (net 7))
 (segment (start 193.53 51.75) (end 194.13 51.75) (width 0.25) (layer F.Cu) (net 7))
 (segment (start 194.13 51.75) (end 194.782501 52.402501) (width 0.25) (layer F.Cu) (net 7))
 (segment (start 192.944998 54.25) (end 193.53 54.25) (width 0.25) (layer F.Cu) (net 7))
 (segment (start 192.694998 54.5) (end 192.944998 54.25) (width 0.25) (layer F.Cu) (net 7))
 (segment (start 192.23 54.5) (end 192.694998 54.5) (width 0.25) (layer F.Cu) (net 7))
 (segment (start 193.485 36) (end 196 36) (width 0.25) (layer F.Cu) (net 8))
 (segment (start 176 52.685) (end 176 54.2) (width 0.25) (layer F.Cu) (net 9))
 (segment (start 176 54.2) (end 176.6 54.8) (width 0.25) (layer F.Cu) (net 9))
 (segment (start 176.6 54.8) (end 178.2 54.8) (width 0.25) (layer F.Cu) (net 9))
 (segment (start 178.2 54.8) (end 178.8 54.2) (width 0.25) (layer F.Cu) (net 9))
 (segment (start 178.8 53.275) (end 179.825 52.25) (width 0.25) (layer F.Cu) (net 9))
 (segment (start 178.8 54.2) (end 178.8 53.275) (width 0.25) (layer F.Cu) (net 9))
 (segment (start 177.2 50.285) (end 177.2 51.715) (width 0.25) (layer F.Cu) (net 10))
 (segment (start 177.315 51.6) (end 177.2 51.715) (width 0.25) (layer F.Cu) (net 10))
 (segment (start 179.825 51.6) (end 177.315 51.6) (width 0.25) (layer F.Cu) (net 10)))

